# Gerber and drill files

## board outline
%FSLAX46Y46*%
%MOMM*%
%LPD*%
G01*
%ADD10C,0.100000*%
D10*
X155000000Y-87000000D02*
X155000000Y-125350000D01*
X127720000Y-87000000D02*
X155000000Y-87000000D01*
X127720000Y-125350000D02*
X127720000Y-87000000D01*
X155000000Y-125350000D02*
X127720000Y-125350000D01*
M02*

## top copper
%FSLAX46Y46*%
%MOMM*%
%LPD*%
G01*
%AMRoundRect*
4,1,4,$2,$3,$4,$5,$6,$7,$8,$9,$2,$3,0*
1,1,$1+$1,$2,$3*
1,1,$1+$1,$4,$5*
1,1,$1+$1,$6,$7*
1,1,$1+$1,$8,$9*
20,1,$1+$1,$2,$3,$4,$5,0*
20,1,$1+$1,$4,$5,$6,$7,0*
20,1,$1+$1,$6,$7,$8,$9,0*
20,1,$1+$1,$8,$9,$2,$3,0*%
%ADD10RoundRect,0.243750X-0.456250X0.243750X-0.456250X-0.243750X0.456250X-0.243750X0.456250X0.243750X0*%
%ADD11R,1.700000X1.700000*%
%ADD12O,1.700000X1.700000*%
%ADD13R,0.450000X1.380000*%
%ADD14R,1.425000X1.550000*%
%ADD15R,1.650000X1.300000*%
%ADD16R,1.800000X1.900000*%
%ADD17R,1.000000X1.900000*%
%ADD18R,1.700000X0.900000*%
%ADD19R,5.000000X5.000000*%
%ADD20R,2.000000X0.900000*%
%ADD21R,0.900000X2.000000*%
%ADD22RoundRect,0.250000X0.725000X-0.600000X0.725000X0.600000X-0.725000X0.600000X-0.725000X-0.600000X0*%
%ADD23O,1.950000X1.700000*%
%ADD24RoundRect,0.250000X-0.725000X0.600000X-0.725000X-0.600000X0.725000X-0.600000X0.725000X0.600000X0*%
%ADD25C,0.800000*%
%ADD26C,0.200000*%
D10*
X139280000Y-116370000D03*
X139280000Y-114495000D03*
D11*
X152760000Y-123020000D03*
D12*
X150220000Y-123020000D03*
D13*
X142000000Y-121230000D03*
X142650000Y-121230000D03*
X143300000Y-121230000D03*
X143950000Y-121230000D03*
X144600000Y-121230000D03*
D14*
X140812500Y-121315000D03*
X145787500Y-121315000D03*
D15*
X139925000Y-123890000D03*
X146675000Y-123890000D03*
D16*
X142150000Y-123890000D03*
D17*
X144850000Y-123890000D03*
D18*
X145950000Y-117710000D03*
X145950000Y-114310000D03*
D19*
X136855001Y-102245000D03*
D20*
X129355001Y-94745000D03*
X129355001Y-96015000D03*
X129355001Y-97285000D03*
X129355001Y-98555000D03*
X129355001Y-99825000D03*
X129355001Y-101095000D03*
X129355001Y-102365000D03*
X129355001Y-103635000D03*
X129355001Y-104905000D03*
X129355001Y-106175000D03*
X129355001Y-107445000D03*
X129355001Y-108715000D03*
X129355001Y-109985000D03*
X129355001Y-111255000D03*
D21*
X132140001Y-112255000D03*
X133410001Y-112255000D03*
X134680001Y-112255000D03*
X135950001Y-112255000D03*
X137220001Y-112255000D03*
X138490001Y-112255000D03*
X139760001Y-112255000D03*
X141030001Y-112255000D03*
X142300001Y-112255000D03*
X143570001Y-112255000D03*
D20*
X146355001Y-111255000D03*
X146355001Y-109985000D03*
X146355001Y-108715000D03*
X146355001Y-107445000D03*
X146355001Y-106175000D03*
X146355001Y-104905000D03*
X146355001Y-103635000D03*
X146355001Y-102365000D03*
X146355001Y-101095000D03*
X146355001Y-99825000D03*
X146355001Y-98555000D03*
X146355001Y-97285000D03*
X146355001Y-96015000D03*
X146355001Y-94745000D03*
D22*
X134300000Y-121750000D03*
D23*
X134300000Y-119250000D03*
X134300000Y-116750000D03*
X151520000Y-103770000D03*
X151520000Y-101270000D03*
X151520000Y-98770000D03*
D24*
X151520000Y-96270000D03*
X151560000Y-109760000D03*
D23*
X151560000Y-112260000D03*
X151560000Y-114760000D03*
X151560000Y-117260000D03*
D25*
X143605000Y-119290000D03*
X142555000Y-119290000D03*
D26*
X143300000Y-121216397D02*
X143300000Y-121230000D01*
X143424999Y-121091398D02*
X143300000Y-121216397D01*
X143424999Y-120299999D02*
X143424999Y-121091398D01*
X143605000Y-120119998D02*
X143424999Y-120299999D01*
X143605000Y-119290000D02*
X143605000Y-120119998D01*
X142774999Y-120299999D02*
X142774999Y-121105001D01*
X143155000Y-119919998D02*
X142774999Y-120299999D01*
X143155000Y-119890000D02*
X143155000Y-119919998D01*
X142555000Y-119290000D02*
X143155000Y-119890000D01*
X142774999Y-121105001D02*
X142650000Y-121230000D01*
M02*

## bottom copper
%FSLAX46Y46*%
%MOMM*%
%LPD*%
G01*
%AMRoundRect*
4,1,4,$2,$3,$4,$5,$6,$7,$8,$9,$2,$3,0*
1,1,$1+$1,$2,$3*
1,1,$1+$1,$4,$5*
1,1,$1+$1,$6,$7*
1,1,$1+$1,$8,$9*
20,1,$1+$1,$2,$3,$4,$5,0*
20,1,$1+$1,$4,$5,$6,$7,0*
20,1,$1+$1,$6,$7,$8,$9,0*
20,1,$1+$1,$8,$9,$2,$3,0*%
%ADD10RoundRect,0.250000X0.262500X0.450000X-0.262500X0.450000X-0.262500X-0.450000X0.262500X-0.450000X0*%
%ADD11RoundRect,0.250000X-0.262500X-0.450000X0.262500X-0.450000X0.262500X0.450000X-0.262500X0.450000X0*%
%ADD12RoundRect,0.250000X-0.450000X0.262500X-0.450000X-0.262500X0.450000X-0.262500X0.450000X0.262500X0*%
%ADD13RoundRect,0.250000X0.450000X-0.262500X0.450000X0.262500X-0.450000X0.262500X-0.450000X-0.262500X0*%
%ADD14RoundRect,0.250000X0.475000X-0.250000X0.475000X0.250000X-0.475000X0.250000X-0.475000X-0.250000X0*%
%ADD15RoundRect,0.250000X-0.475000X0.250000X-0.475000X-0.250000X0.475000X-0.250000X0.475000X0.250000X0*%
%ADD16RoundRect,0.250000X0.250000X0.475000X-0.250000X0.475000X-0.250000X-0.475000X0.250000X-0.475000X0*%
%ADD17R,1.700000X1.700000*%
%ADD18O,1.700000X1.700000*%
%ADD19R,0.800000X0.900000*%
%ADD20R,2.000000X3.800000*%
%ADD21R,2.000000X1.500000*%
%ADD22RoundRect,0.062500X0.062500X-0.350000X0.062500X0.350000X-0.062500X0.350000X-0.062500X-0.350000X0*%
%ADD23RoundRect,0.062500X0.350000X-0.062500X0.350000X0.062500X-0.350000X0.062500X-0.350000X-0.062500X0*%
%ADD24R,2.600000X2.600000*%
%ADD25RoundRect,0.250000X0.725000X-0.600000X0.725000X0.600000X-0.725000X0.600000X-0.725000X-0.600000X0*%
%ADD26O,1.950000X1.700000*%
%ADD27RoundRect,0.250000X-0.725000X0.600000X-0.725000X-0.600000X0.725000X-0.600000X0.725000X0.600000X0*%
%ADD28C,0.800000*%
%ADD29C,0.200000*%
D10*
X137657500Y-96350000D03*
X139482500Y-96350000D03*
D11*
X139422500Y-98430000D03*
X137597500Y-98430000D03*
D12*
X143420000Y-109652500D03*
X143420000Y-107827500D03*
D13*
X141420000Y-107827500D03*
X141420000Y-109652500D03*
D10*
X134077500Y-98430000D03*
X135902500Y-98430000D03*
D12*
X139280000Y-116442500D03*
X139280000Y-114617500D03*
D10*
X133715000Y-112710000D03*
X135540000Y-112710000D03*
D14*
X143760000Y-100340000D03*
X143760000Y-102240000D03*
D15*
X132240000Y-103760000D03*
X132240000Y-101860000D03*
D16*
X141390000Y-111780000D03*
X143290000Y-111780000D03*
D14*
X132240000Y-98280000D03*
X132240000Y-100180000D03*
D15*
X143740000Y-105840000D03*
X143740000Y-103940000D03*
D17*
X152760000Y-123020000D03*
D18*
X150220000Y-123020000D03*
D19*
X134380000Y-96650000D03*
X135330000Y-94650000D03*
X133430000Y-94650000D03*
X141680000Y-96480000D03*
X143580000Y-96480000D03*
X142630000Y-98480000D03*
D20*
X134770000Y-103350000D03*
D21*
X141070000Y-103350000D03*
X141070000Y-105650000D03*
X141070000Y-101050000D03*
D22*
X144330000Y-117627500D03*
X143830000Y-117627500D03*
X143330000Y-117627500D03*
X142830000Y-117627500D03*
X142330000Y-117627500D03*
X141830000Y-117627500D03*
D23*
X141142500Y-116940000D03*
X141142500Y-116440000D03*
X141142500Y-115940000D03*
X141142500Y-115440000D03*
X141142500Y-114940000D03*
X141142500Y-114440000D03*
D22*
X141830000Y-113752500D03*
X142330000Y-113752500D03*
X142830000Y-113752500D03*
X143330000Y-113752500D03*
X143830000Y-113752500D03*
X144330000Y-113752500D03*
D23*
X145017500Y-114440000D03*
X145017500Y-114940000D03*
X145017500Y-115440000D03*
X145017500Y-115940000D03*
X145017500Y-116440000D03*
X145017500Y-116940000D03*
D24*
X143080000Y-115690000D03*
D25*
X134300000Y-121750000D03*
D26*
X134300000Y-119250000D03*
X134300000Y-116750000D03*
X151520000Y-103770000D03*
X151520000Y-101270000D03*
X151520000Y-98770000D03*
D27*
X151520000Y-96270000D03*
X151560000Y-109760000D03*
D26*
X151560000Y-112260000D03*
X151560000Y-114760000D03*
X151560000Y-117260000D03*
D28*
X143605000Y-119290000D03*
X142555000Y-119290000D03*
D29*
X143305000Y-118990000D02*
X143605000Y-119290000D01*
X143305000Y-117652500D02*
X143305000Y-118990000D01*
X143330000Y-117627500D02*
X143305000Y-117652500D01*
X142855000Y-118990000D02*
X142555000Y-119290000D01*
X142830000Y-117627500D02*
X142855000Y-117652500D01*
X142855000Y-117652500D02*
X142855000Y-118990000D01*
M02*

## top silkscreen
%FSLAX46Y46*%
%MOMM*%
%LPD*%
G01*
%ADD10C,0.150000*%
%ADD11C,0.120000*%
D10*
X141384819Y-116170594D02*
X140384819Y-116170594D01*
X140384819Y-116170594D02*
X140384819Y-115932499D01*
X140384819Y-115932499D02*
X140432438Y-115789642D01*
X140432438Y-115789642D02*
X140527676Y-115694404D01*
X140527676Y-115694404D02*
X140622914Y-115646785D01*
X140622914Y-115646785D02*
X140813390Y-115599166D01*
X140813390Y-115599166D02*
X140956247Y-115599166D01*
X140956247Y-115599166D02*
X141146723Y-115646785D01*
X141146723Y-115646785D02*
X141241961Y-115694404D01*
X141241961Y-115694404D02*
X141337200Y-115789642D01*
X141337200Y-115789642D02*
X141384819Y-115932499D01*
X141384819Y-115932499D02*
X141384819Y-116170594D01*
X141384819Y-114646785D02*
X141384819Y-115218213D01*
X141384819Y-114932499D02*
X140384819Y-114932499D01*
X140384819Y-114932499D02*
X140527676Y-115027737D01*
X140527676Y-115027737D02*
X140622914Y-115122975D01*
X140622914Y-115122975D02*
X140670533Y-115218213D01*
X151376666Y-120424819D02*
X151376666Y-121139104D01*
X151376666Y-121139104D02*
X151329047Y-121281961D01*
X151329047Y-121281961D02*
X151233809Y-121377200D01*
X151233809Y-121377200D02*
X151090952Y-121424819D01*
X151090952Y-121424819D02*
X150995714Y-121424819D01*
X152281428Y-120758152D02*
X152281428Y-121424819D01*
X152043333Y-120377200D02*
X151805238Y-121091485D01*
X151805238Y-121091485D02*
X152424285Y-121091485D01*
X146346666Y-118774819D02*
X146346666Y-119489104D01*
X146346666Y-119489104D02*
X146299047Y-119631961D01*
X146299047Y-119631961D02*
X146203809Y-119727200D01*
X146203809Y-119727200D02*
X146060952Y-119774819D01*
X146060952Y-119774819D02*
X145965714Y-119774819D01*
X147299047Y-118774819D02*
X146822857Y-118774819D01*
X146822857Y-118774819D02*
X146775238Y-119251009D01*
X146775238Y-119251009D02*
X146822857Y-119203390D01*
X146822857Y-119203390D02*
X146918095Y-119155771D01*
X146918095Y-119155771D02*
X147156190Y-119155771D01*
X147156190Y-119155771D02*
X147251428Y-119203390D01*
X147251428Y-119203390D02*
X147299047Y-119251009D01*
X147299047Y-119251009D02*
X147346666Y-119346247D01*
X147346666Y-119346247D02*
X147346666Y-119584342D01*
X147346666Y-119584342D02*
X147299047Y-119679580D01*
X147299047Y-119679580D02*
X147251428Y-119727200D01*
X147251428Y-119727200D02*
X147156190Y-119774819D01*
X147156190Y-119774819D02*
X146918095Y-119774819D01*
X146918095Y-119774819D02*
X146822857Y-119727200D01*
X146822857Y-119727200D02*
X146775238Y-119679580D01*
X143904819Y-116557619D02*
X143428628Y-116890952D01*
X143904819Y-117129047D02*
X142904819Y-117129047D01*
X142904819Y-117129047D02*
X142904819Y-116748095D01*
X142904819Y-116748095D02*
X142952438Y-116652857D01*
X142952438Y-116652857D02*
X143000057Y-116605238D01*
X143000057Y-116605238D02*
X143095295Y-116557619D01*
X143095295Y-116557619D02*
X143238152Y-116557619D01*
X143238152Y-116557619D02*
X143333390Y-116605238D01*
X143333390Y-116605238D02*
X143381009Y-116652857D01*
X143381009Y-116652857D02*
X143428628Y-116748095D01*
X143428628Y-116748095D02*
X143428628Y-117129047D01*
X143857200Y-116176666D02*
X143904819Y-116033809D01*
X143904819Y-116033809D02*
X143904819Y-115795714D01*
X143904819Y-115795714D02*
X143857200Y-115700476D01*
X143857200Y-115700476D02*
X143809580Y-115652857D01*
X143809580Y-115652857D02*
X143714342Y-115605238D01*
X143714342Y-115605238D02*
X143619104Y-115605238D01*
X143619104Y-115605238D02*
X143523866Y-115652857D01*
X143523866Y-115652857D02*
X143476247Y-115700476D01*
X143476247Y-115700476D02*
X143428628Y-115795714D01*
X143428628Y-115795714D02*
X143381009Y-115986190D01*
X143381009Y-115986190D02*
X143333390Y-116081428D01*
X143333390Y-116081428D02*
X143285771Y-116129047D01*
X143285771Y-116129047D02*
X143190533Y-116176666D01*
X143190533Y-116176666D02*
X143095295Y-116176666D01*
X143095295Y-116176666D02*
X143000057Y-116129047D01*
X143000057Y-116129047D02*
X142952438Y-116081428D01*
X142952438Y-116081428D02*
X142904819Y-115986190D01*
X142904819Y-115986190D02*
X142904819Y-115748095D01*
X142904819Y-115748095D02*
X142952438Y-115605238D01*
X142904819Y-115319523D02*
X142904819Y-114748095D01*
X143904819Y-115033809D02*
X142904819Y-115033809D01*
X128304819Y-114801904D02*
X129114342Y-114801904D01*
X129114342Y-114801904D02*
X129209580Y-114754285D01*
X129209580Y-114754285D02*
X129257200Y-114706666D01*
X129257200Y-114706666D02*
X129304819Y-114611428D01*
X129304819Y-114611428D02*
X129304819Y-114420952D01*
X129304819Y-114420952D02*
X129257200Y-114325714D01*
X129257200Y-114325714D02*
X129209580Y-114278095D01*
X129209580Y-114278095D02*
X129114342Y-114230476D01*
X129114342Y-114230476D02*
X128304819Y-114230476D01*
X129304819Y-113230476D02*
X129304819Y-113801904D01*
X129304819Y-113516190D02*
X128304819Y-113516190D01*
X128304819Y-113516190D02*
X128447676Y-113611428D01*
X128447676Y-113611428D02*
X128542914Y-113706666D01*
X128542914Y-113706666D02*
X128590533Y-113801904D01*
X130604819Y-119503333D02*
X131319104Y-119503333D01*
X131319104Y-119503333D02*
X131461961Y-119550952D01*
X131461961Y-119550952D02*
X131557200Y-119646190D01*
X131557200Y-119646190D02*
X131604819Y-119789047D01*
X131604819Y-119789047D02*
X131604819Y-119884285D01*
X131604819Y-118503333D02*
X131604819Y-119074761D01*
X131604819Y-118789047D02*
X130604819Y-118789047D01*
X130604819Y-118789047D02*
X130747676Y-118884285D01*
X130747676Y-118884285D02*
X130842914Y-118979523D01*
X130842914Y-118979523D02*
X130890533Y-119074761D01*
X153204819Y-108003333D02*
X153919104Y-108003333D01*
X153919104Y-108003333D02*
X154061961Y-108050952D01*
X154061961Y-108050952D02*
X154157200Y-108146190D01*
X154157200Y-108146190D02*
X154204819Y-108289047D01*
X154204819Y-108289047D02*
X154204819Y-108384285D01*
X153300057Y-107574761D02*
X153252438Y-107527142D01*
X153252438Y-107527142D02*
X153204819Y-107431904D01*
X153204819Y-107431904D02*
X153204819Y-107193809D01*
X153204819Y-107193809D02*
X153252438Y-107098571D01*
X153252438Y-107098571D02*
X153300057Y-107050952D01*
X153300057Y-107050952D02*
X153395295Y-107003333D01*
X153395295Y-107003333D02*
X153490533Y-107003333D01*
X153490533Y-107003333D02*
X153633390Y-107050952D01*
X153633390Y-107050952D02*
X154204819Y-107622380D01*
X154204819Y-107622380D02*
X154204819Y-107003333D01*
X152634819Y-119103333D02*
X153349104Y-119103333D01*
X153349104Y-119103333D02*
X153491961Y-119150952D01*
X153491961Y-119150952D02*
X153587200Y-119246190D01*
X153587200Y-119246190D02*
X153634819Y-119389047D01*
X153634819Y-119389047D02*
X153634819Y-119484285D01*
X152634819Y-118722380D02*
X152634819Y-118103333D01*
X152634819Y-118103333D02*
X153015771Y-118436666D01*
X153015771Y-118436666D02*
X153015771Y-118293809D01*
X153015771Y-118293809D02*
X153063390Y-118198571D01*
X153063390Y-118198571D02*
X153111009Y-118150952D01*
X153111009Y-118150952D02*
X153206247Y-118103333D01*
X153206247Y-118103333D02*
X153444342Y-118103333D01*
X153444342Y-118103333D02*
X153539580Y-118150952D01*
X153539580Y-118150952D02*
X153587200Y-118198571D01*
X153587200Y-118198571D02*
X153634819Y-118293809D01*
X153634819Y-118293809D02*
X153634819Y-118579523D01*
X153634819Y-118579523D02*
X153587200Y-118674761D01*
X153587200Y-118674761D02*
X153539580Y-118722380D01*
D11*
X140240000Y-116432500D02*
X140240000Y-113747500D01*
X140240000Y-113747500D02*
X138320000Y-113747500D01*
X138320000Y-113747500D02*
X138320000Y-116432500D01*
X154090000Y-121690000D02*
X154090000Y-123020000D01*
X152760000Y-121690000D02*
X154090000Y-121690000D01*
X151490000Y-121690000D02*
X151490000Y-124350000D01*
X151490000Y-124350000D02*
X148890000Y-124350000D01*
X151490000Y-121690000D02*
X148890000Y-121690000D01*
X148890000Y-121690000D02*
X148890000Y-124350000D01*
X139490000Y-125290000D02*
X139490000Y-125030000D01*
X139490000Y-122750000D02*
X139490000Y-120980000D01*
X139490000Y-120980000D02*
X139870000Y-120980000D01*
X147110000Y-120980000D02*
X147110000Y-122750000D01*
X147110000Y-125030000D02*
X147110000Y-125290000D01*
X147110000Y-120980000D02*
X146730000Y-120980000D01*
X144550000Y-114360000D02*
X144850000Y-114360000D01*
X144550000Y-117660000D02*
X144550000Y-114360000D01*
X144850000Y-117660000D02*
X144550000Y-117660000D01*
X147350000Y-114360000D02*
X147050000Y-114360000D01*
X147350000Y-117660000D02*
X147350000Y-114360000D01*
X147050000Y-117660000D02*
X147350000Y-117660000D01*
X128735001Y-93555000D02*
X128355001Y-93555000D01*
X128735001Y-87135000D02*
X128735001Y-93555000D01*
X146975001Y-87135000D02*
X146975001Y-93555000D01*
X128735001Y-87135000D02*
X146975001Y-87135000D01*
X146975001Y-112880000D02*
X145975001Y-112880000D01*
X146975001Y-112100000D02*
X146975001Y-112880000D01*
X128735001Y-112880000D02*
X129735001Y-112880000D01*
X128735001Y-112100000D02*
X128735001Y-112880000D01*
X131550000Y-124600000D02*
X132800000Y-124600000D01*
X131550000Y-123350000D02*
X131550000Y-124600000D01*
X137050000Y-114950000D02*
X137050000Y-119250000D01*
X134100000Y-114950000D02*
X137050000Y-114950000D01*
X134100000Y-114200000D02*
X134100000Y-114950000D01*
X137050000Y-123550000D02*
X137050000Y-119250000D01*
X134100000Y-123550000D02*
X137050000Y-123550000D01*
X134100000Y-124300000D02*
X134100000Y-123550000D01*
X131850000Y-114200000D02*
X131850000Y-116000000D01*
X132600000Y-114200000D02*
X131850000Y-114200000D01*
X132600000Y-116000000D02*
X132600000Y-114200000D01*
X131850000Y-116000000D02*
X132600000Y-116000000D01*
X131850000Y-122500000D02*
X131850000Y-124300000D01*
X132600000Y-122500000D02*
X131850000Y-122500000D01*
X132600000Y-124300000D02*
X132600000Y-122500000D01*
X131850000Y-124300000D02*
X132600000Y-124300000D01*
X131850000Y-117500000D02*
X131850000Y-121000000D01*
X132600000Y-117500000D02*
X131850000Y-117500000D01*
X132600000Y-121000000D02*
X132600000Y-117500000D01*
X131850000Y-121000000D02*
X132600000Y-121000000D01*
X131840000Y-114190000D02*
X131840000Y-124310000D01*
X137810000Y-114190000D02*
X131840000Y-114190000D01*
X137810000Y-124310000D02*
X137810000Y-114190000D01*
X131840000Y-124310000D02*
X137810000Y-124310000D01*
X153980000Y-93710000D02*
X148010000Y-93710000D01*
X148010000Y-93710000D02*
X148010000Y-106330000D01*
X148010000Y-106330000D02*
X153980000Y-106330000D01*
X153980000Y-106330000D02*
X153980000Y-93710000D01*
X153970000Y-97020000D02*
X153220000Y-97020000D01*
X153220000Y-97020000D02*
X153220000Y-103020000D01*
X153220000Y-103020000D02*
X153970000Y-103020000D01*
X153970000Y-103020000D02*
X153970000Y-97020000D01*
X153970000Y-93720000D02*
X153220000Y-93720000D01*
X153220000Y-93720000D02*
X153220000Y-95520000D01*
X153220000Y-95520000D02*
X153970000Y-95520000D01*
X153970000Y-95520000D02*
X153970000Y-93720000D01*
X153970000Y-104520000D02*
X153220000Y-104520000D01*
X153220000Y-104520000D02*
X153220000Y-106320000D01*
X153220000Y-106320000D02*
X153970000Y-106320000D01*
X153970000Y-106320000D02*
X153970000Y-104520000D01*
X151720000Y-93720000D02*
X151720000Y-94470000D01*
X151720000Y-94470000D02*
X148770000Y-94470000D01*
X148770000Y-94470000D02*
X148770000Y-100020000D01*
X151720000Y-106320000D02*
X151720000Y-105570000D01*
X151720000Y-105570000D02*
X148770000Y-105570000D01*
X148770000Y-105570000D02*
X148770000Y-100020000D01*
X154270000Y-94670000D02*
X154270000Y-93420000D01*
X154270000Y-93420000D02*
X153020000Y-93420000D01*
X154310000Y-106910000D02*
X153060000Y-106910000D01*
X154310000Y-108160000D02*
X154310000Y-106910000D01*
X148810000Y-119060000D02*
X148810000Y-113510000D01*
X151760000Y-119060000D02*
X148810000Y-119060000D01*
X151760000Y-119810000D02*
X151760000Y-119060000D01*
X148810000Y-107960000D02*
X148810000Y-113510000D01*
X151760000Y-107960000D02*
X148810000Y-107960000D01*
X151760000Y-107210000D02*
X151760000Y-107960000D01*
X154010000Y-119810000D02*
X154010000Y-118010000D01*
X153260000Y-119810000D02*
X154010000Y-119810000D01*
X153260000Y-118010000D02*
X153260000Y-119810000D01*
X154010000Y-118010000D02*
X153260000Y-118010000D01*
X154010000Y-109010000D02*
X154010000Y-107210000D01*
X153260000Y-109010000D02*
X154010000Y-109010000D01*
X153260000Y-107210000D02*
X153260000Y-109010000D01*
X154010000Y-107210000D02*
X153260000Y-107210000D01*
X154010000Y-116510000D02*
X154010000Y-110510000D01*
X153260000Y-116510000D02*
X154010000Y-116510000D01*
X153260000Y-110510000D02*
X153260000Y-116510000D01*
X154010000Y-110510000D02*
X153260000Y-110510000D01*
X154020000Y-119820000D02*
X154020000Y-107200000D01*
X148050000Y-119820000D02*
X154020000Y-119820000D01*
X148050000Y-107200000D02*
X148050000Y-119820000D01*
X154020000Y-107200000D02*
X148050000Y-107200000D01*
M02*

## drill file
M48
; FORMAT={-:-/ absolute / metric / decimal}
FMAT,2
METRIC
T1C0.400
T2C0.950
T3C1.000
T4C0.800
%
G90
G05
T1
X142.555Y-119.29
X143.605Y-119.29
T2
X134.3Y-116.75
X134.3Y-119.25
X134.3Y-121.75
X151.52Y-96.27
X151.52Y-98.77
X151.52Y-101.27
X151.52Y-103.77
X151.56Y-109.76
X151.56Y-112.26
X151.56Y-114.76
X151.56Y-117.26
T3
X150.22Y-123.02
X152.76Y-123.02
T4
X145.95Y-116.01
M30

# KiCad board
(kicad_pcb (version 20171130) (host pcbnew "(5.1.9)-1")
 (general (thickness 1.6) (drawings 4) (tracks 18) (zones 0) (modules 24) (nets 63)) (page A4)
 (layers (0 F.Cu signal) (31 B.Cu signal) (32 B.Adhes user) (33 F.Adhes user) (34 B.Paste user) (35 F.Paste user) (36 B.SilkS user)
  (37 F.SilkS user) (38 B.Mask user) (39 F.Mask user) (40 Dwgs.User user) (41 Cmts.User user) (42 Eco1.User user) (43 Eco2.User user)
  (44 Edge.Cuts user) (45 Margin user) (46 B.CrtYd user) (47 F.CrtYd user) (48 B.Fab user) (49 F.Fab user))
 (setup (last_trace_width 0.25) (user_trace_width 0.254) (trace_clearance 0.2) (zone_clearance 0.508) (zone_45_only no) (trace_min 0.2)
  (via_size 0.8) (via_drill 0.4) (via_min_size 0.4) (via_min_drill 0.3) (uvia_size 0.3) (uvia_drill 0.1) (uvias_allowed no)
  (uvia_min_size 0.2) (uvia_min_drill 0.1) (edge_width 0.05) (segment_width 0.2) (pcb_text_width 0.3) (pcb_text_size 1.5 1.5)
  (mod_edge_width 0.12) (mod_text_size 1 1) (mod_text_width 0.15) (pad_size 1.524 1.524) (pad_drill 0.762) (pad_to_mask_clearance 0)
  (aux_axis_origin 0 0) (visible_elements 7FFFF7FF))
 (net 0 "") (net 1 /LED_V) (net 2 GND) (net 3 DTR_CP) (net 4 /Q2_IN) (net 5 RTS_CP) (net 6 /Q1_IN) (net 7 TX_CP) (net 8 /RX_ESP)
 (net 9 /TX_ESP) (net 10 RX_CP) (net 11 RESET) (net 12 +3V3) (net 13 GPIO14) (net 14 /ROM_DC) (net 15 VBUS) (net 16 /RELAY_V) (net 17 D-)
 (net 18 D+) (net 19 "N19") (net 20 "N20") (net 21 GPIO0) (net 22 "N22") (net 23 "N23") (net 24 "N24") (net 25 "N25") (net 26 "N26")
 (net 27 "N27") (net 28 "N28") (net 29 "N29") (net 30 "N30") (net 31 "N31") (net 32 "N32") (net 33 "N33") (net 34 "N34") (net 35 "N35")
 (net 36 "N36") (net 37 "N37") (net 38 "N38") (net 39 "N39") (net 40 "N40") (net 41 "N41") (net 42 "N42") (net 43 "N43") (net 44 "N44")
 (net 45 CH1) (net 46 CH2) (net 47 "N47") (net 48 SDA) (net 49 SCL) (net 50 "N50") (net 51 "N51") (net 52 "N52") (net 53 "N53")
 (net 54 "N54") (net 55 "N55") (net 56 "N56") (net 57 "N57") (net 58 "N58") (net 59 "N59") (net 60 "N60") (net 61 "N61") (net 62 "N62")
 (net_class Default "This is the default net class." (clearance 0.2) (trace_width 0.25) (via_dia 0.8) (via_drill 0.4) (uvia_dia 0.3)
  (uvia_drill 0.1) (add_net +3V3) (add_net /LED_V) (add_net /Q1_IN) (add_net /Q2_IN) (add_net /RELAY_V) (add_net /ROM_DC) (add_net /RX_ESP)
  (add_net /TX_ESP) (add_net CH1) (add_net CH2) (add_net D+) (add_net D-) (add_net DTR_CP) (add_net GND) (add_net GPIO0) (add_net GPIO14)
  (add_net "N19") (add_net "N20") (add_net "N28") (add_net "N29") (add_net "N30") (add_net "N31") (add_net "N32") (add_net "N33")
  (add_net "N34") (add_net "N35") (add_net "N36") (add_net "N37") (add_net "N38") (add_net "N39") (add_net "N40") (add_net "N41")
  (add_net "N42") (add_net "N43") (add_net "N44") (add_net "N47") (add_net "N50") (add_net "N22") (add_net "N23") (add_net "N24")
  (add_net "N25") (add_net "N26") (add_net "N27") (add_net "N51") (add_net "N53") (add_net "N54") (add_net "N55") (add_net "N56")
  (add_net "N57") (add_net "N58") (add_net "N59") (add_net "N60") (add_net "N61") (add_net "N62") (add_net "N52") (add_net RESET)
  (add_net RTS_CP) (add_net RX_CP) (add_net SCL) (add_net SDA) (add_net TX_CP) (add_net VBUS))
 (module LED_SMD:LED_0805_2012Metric (layer F.Cu) (at 139.28 115.4325 270)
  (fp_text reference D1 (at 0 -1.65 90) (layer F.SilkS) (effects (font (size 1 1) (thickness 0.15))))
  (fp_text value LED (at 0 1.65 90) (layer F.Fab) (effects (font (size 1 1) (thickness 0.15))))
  (fp_line (start 1 -0.96) (end -1.685 -0.96) (layer F.SilkS) (width 0.12))
  (fp_line (start -1.685 -0.96) (end -1.685 0.96) (layer F.SilkS) (width 0.12))
  (fp_line (start -1.685 0.96) (end 1 0.96) (layer F.SilkS) (width 0.12))
  (pad 2 smd roundrect (at 0.9375 0 270) (size 0.975 1.4) (layers F.Cu F.Paste F.Mask) (roundrect_rratio 0.25) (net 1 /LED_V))
  (pad 1 smd roundrect (at -0.9375 0 270) (size 0.975 1.4) (layers F.Cu F.Paste F.Mask) (roundrect_rratio 0.25) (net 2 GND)))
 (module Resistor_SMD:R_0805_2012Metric (layer B.Cu) (at 138.57 96.35 180)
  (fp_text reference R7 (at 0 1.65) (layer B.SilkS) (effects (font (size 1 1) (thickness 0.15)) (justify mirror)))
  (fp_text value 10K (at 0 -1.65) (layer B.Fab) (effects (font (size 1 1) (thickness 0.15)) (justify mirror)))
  (pad 2 smd roundrect (at 0.9125 0 180) (size 1.025 1.4) (layers B.Cu B.Paste B.Mask) (roundrect_rratio 0.243902) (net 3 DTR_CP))
  (pad 1 smd roundrect (at -0.9125 0 180) (size 1.025 1.4) (layers B.Cu B.Paste B.Mask) (roundrect_rratio 0.243902) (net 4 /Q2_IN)))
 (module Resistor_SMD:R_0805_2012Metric (layer B.Cu) (at 138.51 98.43)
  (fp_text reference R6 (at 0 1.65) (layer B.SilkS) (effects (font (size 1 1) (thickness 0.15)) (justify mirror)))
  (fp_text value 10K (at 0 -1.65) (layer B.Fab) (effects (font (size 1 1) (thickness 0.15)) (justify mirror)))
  (pad 2 smd roundrect (at 0.9125 0) (size 1.025 1.4) (layers B.Cu B.Paste B.Mask) (roundrect_rratio 0.243902) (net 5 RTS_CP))
  (pad 1 smd roundrect (at -0.9125 0) (size 1.025 1.4) (layers B.Cu B.Paste B.Mask) (roundrect_rratio 0.243902) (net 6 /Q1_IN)))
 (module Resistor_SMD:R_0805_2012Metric (layer B.Cu) (at 143.42 108.74 270)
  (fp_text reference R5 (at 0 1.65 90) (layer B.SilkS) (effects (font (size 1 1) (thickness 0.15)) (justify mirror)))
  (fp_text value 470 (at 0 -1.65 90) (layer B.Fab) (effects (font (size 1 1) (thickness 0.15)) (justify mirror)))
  (pad 2 smd roundrect (at 0.9125 0 270) (size 1.025 1.4) (layers B.Cu B.Paste B.Mask) (roundrect_rratio 0.243902) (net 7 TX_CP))
  (pad 1 smd roundrect (at -0.9125 0 270) (size 1.025 1.4) (layers B.Cu B.Paste B.Mask) (roundrect_rratio 0.243902) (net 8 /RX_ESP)))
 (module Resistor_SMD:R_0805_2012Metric (layer B.Cu) (at 141.42 108.74 90)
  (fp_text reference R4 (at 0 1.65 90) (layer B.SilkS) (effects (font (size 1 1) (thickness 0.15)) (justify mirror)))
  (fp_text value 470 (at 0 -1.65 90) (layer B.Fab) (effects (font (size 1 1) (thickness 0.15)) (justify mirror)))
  (pad 2 smd roundrect (at 0.9125 0 90) (size 1.025 1.4) (layers B.Cu B.Paste B.Mask) (roundrect_rratio 0.243902) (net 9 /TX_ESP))
  (pad 1 smd roundrect (at -0.9125 0 90) (size 1.025 1.4) (layers B.Cu B.Paste B.Mask) (roundrect_rratio 0.243902) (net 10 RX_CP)))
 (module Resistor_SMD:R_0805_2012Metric (layer B.Cu) (at 134.99 98.43 180)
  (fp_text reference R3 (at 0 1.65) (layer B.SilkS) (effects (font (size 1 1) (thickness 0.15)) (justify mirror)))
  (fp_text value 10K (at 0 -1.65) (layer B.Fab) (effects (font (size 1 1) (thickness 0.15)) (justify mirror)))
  (pad 2 smd roundrect (at 0.9125 0 180) (size 1.025 1.4) (layers B.Cu B.Paste B.Mask) (roundrect_rratio 0.243902) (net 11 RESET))
  (pad 1 smd roundrect (at -0.9125 0 180) (size 1.025 1.4) (layers B.Cu B.Paste B.Mask) (roundrect_rratio 0.243902) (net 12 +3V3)))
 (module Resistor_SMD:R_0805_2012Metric (layer B.Cu) (at 139.28 115.53 270)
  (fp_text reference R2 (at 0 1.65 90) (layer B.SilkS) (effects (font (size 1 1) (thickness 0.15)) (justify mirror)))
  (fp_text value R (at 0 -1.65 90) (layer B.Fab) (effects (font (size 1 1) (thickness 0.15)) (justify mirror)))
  (pad 2 smd roundrect (at 0.9125 0 270) (size 1.025 1.4) (layers B.Cu B.Paste B.Mask) (roundrect_rratio 0.243902) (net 1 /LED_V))
  (pad 1 smd roundrect (at -0.9125 0 270) (size 1.025 1.4) (layers B.Cu B.Paste B.Mask) (roundrect_rratio 0.243902) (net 12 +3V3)))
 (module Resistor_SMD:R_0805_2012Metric (layer B.Cu) (at 134.6275 112.71 180)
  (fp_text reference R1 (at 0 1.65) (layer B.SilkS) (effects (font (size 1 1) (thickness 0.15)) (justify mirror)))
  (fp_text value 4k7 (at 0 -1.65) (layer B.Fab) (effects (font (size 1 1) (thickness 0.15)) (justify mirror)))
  (pad 2 smd roundrect (at 0.9125 0 180) (size 1.025 1.4) (layers B.Cu B.Paste B.Mask) (roundrect_rratio 0.243902) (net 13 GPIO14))
  (pad 1 smd roundrect (at -0.9125 0 180) (size 1.025 1.4) (layers B.Cu B.Paste B.Mask) (roundrect_rratio 0.243902) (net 12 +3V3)))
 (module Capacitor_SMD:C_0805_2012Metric (layer B.Cu) (at 143.76 101.29 90)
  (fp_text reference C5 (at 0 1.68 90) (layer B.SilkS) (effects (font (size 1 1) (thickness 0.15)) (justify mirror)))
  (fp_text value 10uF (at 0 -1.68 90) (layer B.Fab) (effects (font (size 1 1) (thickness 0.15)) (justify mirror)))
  (pad 2 smd roundrect (at 0.95 0 90) (size 1 1.45) (layers B.Cu B.Paste B.Mask) (roundrect_rratio 0.25) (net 2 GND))
  (pad 1 smd roundrect (at -0.95 0 90) (size 1 1.45) (layers B.Cu B.Paste B.Mask) (roundrect_rratio 0.25) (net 12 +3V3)))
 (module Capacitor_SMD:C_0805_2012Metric (layer B.Cu) (at 132.24 102.81 270)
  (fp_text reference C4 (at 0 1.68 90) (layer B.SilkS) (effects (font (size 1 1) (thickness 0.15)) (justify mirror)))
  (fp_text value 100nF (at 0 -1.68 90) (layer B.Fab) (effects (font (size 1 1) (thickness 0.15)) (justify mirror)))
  (pad 2 smd roundrect (at 0.95 0 270) (size 1 1.45) (layers B.Cu B.Paste B.Mask) (roundrect_rratio 0.25) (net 12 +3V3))
  (pad 1 smd roundrect (at -0.95 0 270) (size 1 1.45) (layers B.Cu B.Paste B.Mask) (roundrect_rratio 0.25) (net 2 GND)))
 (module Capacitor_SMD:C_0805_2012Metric (layer B.Cu) (at 142.34 111.78 180)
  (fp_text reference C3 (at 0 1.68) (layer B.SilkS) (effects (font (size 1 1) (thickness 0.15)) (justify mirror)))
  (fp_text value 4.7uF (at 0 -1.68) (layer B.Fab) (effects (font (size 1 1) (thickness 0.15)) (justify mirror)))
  (pad 2 smd roundrect (at 0.95 0 180) (size 1 1.45) (layers B.Cu B.Paste B.Mask) (roundrect_rratio 0.25) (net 2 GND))
  (pad 1 smd roundrect (at -0.95 0 180) (size 1 1.45) (layers B.Cu B.Paste B.Mask) (roundrect_rratio 0.25) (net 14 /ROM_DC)))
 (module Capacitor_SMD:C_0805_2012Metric (layer B.Cu) (at 132.24 99.23 90)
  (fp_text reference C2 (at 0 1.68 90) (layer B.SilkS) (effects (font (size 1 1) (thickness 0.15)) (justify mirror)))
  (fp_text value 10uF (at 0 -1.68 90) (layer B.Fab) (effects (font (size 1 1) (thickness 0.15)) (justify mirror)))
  (pad 2 smd roundrect (at 0.95 0 90) (size 1 1.45) (layers B.Cu B.Paste B.Mask) (roundrect_rratio 0.25) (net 11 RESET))
  (pad 1 smd roundrect (at -0.95 0 90) (size 1 1.45) (layers B.Cu B.Paste B.Mask) (roundrect_rratio 0.25) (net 2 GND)))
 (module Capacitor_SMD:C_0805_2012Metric (layer B.Cu) (at 143.74 104.89 270)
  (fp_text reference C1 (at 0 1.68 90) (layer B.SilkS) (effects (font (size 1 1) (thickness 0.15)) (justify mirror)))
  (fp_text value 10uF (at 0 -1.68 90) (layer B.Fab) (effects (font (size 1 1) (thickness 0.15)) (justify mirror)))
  (pad 2 smd roundrect (at 0.95 0 270) (size 1 1.45) (layers B.Cu B.Paste B.Mask) (roundrect_rratio 0.25) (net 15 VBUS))
  (pad 1 smd roundrect (at -0.95 0 270) (size 1 1.45) (layers B.Cu B.Paste B.Mask) (roundrect_rratio 0.25) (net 2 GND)))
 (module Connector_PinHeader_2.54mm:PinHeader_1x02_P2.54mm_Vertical (layer F.Cu) (at 152.76 123.02 270)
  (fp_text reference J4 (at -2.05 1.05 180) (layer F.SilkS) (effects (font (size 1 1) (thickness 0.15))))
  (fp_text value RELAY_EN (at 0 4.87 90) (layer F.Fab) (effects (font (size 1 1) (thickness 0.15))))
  (fp_line (start -1.33 -1.33) (end 0 -1.33) (layer F.SilkS) (width 0.12))
  (fp_line (start -1.33 0) (end -1.33 -1.33) (layer F.SilkS) (width 0.12))
  (fp_line (start -1.33 1.27) (end 1.33 1.27) (layer F.SilkS) (width 0.12))
  (fp_line (start 1.33 1.27) (end 1.33 3.87) (layer F.SilkS) (width 0.12))
  (fp_line (start -1.33 1.27) (end -1.33 3.87) (layer F.SilkS) (width 0.12))
  (fp_line (start -1.33 3.87) (end 1.33 3.87) (layer F.SilkS) (width 0.12))
  (pad 1 thru_hole rect (at 0 0 270) (size 1.7 1.7) (drill 1) (layers *.Cu *.Mask) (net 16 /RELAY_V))
  (pad 2 thru_hole oval (at 0 2.54 270) (size 1.7 1.7) (drill 1) (layers *.Cu *.Mask) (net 15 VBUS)))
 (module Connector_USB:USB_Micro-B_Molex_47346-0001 (layer F.Cu) (at 143.3 122.69)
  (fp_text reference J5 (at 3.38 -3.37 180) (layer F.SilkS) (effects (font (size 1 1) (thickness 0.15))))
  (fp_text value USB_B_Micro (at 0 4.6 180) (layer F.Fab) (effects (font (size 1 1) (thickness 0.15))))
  (fp_line (start -3.81 2.6) (end -3.81 2.34) (layer F.SilkS) (width 0.12))
  (fp_line (start -3.81 0.06) (end -3.81 -1.71) (layer F.SilkS) (width 0.12))
  (fp_line (start -3.81 -1.71) (end -3.43 -1.71) (layer F.SilkS) (width 0.12))
  (fp_line (start 3.81 -1.71) (end 3.81 0.06) (layer F.SilkS) (width 0.12))
  (fp_line (start 3.81 2.34) (end 3.81 2.6) (layer F.SilkS) (width 0.12))
  (fp_line (start 3.81 -1.71) (end 3.43 -1.71) (layer F.SilkS) (width 0.12))
  (pad 1 smd rect (at -1.3 -1.46) (size 0.45 1.38) (layers F.Cu F.Paste F.Mask) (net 15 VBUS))
  (pad 2 smd rect (at -0.65 -1.46) (size 0.45 1.38) (layers F.Cu F.Paste F.Mask) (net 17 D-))
  (pad 3 smd rect (at 0 -1.46) (size 0.45 1.38) (layers F.Cu F.Paste F.Mask) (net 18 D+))
  (pad 4 smd rect (at 0.65 -1.46) (size 0.45 1.38) (layers F.Cu F.Paste F.Mask) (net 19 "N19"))
  (pad 5 smd rect (at 1.3 -1.46) (size 0.45 1.38) (layers F.Cu F.Paste F.Mask) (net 2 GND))
  (pad 6 smd rect (at -2.4875 -1.375) (size 1.425 1.55) (layers F.Cu F.Paste F.Mask) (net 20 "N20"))
  (pad 6 smd rect (at 2.4875 -1.375) (size 1.425 1.55) (layers F.Cu F.Paste F.Mask) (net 20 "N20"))
  (pad 6 smd rect (at -3.375 1.2) (size 1.65 1.3) (layers F.Cu F.Paste F.Mask) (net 20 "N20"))
  (pad 6 smd rect (at 3.375 1.2) (size 1.65 1.3) (layers F.Cu F.Paste F.Mask) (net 20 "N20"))
  (pad 6 smd rect (at -1.15 1.2) (size 1.8 1.9) (layers F.Cu F.Paste F.Mask) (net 20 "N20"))
  (pad 6 smd rect (at 1.55 1.2) (size 1 1.9) (layers F.Cu F.Paste F.Mask) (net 20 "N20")))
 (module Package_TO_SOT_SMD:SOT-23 (layer B.Cu) (at 134.38 95.65 270)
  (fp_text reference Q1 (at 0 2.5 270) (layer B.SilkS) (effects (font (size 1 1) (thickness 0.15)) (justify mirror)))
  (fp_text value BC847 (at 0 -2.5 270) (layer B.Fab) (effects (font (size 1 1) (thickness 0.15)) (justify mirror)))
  (pad 3 smd rect (at 1 0 270) (size 0.9 0.8) (layers B.Cu B.Paste B.Mask) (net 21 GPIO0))
  (pad 2 smd rect (at -1 -0.95 270) (size 0.9 0.8) (layers B.Cu B.Paste B.Mask) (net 3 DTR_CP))
  (pad 1 smd rect (at -1 0.95 270) (size 0.9 0.8) (layers B.Cu B.Paste B.Mask) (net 6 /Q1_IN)))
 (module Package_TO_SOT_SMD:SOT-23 (layer B.Cu) (at 142.63 97.48 270)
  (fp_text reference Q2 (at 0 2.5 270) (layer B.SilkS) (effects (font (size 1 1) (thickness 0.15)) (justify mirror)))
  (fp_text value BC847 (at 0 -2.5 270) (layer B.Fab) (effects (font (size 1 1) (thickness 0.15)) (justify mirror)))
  (pad 1 smd rect (at -1 0.95 270) (size 0.9 0.8) (layers B.Cu B.Paste B.Mask) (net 4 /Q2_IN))
  (pad 2 smd rect (at -1 -0.95 270) (size 0.9 0.8) (layers B.Cu B.Paste B.Mask) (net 11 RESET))
  (pad 3 smd rect (at 1 0 270) (size 0.9 0.8) (layers B.Cu B.Paste B.Mask) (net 5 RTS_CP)))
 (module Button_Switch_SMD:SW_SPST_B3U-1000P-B (layer F.Cu) (at 145.95 116.01 90)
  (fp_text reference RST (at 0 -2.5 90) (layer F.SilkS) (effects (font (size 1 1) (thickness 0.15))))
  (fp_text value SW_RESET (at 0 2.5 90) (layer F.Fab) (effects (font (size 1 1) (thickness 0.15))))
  (fp_line (start 1.65 -1.4) (end 1.65 -1.1) (layer F.SilkS) (width 0.12))
  (fp_line (start -1.65 -1.4) (end 1.65 -1.4) (layer F.SilkS) (width 0.12))
  (fp_line (start -1.65 -1.1) (end -1.65 -1.4) (layer F.SilkS) (width 0.12))
  (fp_line (start 1.65 1.4) (end 1.65 1.1) (layer F.SilkS) (width 0.12))
  (fp_line (start -1.65 1.4) (end 1.65 1.4) (layer F.SilkS) (width 0.12))
  (fp_line (start -1.65 1.1) (end -1.65 1.4) (layer F.SilkS) (width 0.12))
  (pad 1 smd rect (at -1.7 0 90) (size 0.9 1.7) (layers F.Cu F.Paste F.Mask) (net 2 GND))
  (pad 2 smd rect (at 1.7 0 90) (size 0.9 1.7) (layers F.Cu F.Paste F.Mask) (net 11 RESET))
  (pad "" np_thru_hole circle (at 0 0 90) (size 0.8 0.8) (drill 0.8) (layers *.Cu *.Mask)))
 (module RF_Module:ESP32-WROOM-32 (layer F.Cu) (at 137.855001 103)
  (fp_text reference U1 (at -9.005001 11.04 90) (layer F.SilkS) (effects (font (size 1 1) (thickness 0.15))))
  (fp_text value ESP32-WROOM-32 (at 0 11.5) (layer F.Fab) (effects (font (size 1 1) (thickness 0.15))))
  (fp_line (start -9.12 -9.445) (end -9.5 -9.445) (layer F.SilkS) (width 0.12))
  (fp_line (start -9.12 -15.865) (end -9.12 -9.445) (layer F.SilkS) (width 0.12))
  (fp_line (start 9.12 -15.865) (end 9.12 -9.445) (layer F.SilkS) (width 0.12))
  (fp_line (start -9.12 -15.865) (end 9.12 -15.865) (layer F.SilkS) (width 0.12))
  (fp_line (start 9.12 9.88) (end 8.12 9.88) (layer F.SilkS) (width 0.12))
  (fp_line (start 9.12 9.1) (end 9.12 9.88) (layer F.SilkS) (width 0.12))
  (fp_line (start -9.12 9.88) (end -8.12 9.88) (layer F.SilkS) (width 0.12))
  (fp_line (start -9.12 9.1) (end -9.12 9.88) (layer F.SilkS) (width 0.12))
  (pad 39 smd rect (at -1 -0.755) (size 5 5) (layers F.Cu F.Paste F.Mask) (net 2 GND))
  (pad 1 smd rect (at -8.5 -8.255) (size 2 0.9) (layers F.Cu F.Paste F.Mask) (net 2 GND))
  (pad 2 smd rect (at -8.5 -6.985) (size 2 0.9) (layers F.Cu F.Paste F.Mask) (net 12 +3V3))
  (pad 3 smd rect (at -8.5 -5.715) (size 2 0.9) (layers F.Cu F.Paste F.Mask) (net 11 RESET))
  (pad 4 smd rect (at -8.5 -4.445) (size 2 0.9) (layers F.Cu F.Paste F.Mask) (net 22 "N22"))
  (pad 5 smd rect (at -8.5 -3.175) (size 2 0.9) (layers F.Cu F.Paste F.Mask) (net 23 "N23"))
  (pad 6 smd rect (at -8.5 -1.905) (size 2 0.9) (layers F.Cu F.Paste F.Mask) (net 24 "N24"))
  (pad 7 smd rect (at -8.5 -0.635) (size 2 0.9) (layers F.Cu F.Paste F.Mask) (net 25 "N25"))
  (pad 8 smd rect (at -8.5 0.635) (size 2 0.9) (layers F.Cu F.Paste F.Mask) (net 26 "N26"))
  (pad 9 smd rect (at -8.5 1.905) (size 2 0.9) (layers F.Cu F.Paste F.Mask) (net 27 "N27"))
  (pad 10 smd rect (at -8.5 3.175) (size 2 0.9) (layers F.Cu F.Paste F.Mask) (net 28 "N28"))
  (pad 11 smd rect (at -8.5 4.445) (size 2 0.9) (layers F.Cu F.Paste F.Mask) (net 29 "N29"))
  (pad 12 smd rect (at -8.5 5.715) (size 2 0.9) (layers F.Cu F.Paste F.Mask) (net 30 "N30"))
  (pad 13 smd rect (at -8.5 6.985) (size 2 0.9) (layers F.Cu F.Paste F.Mask) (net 13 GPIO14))
  (pad 14 smd rect (at -8.5 8.255) (size 2 0.9) (layers F.Cu F.Paste F.Mask) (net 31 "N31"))
  (pad 15 smd rect (at -5.715 9.255 90) (size 2 0.9) (layers F.Cu F.Paste F.Mask) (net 2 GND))
  (pad 16 smd rect (at -4.445 9.255 90) (size 2 0.9) (layers F.Cu F.Paste F.Mask) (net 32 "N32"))
  (pad 17 smd rect (at -3.175 9.255 90) (size 2 0.9) (layers F.Cu F.Paste F.Mask) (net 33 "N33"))
  (pad 18 smd rect (at -1.905 9.255 90) (size 2 0.9) (layers F.Cu F.Paste F.Mask) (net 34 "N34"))
  (pad 19 smd rect (at -0.635 9.255 90) (size 2 0.9) (layers F.Cu F.Paste F.Mask) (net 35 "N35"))
  (pad 20 smd rect (at 0.635 9.255 90) (size 2 0.9) (layers F.Cu F.Paste F.Mask) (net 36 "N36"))
  (pad 21 smd rect (at 1.905 9.255 90) (size 2 0.9) (layers F.Cu F.Paste F.Mask) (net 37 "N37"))
  (pad 22 smd rect (at 3.175 9.255 90) (size 2 0.9) (layers F.Cu F.Paste F.Mask) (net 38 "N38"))
  (pad 23 smd rect (at 4.445 9.255 90) (size 2 0.9) (layers F.Cu F.Paste F.Mask) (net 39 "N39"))
  (pad 24 smd rect (at 5.715 9.255 90) (size 2 0.9) (layers F.Cu F.Paste F.Mask) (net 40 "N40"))
  (pad 25 smd rect (at 8.5 8.255) (size 2 0.9) (layers F.Cu F.Paste F.Mask) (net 21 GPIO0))
  (pad 26 smd rect (at 8.5 6.985) (size 2 0.9) (layers F.Cu F.Paste F.Mask) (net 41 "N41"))
  (pad 27 smd rect (at 8.5 5.715) (size 2 0.9) (layers F.Cu F.Paste F.Mask) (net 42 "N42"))
  (pad 28 smd rect (at 8.5 4.445) (size 2 0.9) (layers F.Cu F.Paste F.Mask) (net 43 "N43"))
  (pad 29 smd rect (at 8.5 3.175) (size 2 0.9) (layers F.Cu F.Paste F.Mask) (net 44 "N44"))
  (pad 30 smd rect (at 8.5 1.905) (size 2 0.9) (layers F.Cu F.Paste F.Mask) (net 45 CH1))
  (pad 31 smd rect (at 8.5 0.635) (size 2 0.9) (layers F.Cu F.Paste F.Mask) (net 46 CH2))
  (pad 32 smd rect (at 8.5 -0.635) (size 2 0.9) (layers F.Cu F.Paste F.Mask) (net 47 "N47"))
  (pad 33 smd rect (at 8.5 -1.905) (size 2 0.9) (layers F.Cu F.Paste F.Mask) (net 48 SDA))
  (pad 34 smd rect (at 8.5 -3.175) (size 2 0.9) (layers F.Cu F.Paste F.Mask) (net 8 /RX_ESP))
  (pad 35 smd rect (at 8.5 -4.445) (size 2 0.9) (layers F.Cu F.Paste F.Mask) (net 9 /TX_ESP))
  (pad 36 smd rect (at 8.5 -5.715) (size 2 0.9) (layers F.Cu F.Paste F.Mask) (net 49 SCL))
  (pad 37 smd rect (at 8.5 -6.985) (size 2 0.9) (layers F.Cu F.Paste F.Mask) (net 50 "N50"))
  (pad 38 smd rect (at 8.5 -8.255) (size 2 0.9) (layers F.Cu F.Paste F.Mask) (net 2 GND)))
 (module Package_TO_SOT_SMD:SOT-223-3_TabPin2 (layer B.Cu) (at 137.92 103.35 180)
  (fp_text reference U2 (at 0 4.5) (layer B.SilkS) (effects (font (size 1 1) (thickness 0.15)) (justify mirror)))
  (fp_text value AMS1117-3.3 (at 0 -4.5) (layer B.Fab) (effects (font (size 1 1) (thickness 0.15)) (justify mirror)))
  (pad 2 smd rect (at 3.15 0 180) (size 2 3.8) (layers B.Cu B.Paste B.Mask) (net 12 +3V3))
  (pad 2 smd rect (at -3.15 0 180) (size 2 1.5) (layers B.Cu B.Paste B.Mask) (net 12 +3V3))
  (pad 3 smd rect (at -3.15 -2.3 180) (size 2 1.5) (layers B.Cu B.Paste B.Mask) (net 15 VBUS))
  (pad 1 smd rect (at -3.15 2.3 180) (size 2 1.5) (layers B.Cu B.Paste B.Mask) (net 2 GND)))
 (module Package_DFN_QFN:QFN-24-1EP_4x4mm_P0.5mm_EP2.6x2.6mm (layer B.Cu) (at 143.08 115.69 90)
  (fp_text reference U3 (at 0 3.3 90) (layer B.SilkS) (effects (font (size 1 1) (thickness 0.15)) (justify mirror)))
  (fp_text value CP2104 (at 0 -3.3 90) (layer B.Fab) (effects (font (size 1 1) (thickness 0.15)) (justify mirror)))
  (pad 1 smd roundrect (at -1.9375 1.25 90) (size 0.825 0.25) (layers B.Cu B.Paste B.Mask) (roundrect_rratio 0.25) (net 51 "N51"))
  (pad 2 smd roundrect (at -1.9375 0.75 90) (size 0.825 0.25) (layers B.Cu B.Paste B.Mask) (roundrect_rratio 0.25) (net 2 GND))
  (pad 3 smd roundrect (at -1.9375 0.25 90) (size 0.825 0.25) (layers B.Cu B.Paste B.Mask) (roundrect_rratio 0.25) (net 18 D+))
  (pad 4 smd roundrect (at -1.9375 -0.25 90) (size 0.825 0.25) (layers B.Cu B.Paste B.Mask) (roundrect_rratio 0.25) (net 17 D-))
  (pad 5 smd roundrect (at -1.9375 -0.75 90) (size 0.825 0.25) (layers B.Cu B.Paste B.Mask) (roundrect_rratio 0.25) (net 12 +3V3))
  (pad 6 smd roundrect (at -1.9375 -1.25 90) (size 0.825 0.25) (layers B.Cu B.Paste B.Mask) (roundrect_rratio 0.25) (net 12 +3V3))
  (pad 7 smd roundrect (at -1.25 -1.9375 90) (size 0.25 0.825) (layers B.Cu B.Paste B.Mask) (roundrect_rratio 0.25) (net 12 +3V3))
  (pad 8 smd roundrect (at -0.75 -1.9375 90) (size 0.25 0.825) (layers B.Cu B.Paste B.Mask) (roundrect_rratio 0.25) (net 15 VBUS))
  (pad 9 smd roundrect (at -0.25 -1.9375 90) (size 0.25 0.825) (layers B.Cu B.Paste B.Mask) (roundrect_rratio 0.25) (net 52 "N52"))
  (pad 10 smd roundrect (at 0.25 -1.9375 90) (size 0.25 0.825) (layers B.Cu B.Paste B.Mask) (roundrect_rratio 0.25) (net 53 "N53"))
  (pad 11 smd roundrect (at 0.75 -1.9375 90) (size 0.25 0.825) (layers B.Cu B.Paste B.Mask) (roundrect_rratio 0.25) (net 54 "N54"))
  (pad 12 smd roundrect (at 1.25 -1.9375 90) (size 0.25 0.825) (layers B.Cu B.Paste B.Mask) (roundrect_rratio 0.25) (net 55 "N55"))
  (pad 13 smd roundrect (at 1.9375 -1.25 90) (size 0.825 0.25) (layers B.Cu B.Paste B.Mask) (roundrect_rratio 0.25) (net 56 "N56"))
  (pad 14 smd roundrect (at 1.9375 -0.75 90) (size 0.825 0.25) (layers B.Cu B.Paste B.Mask) (roundrect_rratio 0.25) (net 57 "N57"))
  (pad 15 smd roundrect (at 1.9375 -0.25 90) (size 0.825 0.25) (layers B.Cu B.Paste B.Mask) (roundrect_rratio 0.25) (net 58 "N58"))
  (pad 16 smd roundrect (at 1.9375 0.25 90) (size 0.825 0.25) (layers B.Cu B.Paste B.Mask) (roundrect_rratio 0.25) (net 14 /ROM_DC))
  (pad 17 smd roundrect (at 1.9375 0.75 90) (size 0.825 0.25) (layers B.Cu B.Paste B.Mask) (roundrect_rratio 0.25) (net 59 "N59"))
  (pad 18 smd roundrect (at 1.9375 1.25 90) (size 0.825 0.25) (layers B.Cu B.Paste B.Mask) (roundrect_rratio 0.25) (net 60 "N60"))
  (pad 19 smd roundrect (at 1.25 1.9375 90) (size 0.25 0.825) (layers B.Cu B.Paste B.Mask) (roundrect_rratio 0.25) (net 5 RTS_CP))
  (pad 20 smd roundrect (at 0.75 1.9375 90) (size 0.25 0.825) (layers B.Cu B.Paste B.Mask) (roundrect_rratio 0.25) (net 10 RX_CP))
  (pad 21 smd roundrect (at 0.25 1.9375 90) (size 0.25 0.825) (layers B.Cu B.Paste B.Mask) (roundrect_rratio 0.25) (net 7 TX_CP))
  (pad 22 smd roundrect (at -0.25 1.9375 90) (size 0.25 0.825) (layers B.Cu B.Paste B.Mask) (roundrect_rratio 0.25) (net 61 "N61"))
  (pad 23 smd roundrect (at -0.75 1.9375 90) (size 0.25 0.825) (layers B.Cu B.Paste B.Mask) (roundrect_rratio 0.25) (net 3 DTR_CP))
  (pad 24 smd roundrect (at -1.25 1.9375 90) (size 0.25 0.825) (layers B.Cu B.Paste B.Mask) (roundrect_rratio 0.25) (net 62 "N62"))
  (pad 25 smd rect (at 0 0 90) (size 2.6 2.6) (layers B.Cu B.Mask) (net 2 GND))
  (pad "" smd roundrect (at -0.65 0.65 90) (size 1.05 1.05) (layers B.Paste) (roundrect_rratio 0.238095))
  (pad "" smd roundrect (at -0.65 -0.65 90) (size 1.05 1.05) (layers B.Paste) (roundrect_rratio 0.238095))
  (pad "" smd roundrect (at 0.65 0.65 90) (size 1.05 1.05) (layers B.Paste) (roundrect_rratio 0.238095))
  (pad "" smd roundrect (at 0.65 -0.65 90) (size 1.05 1.05) (layers B.Paste) (roundrect_rratio 0.238095)))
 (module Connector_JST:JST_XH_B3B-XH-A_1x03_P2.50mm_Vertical (layer F.Cu) (at 134.3 121.75 90)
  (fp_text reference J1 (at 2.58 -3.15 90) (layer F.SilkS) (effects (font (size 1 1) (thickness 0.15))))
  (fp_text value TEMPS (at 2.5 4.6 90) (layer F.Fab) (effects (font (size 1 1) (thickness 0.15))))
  (fp_line (start -2.85 -2.75) (end -2.85 -1.5) (layer F.SilkS) (width 0.12))
  (fp_line (start -1.6 -2.75) (end -2.85 -2.75) (layer F.SilkS) (width 0.12))
  (fp_line (start 6.8 2.75) (end 2.5 2.75) (layer F.SilkS) (width 0.12))
  (fp_line (start 6.8 -0.2) (end 6.8 2.75) (layer F.SilkS) (width 0.12))
  (fp_line (start 7.55 -0.2) (end 6.8 -0.2) (layer F.SilkS) (width 0.12))
  (fp_line (start -1.8 2.75) (end 2.5 2.75) (layer F.SilkS) (width 0.12))
  (fp_line (start -1.8 -0.2) (end -1.8 2.75) (layer F.SilkS) (width 0.12))
  (fp_line (start -2.55 -0.2) (end -1.8 -0.2) (layer F.SilkS) (width 0.12))
  (fp_line (start 7.55 -2.45) (end 5.75 -2.45) (layer F.SilkS) (width 0.12))
  (fp_line (start 7.55 -1.7) (end 7.55 -2.45) (layer F.SilkS) (width 0.12))
  (fp_line (start 5.75 -1.7) (end 7.55 -1.7) (layer F.SilkS) (width 0.12))
  (fp_line (start 5.75 -2.45) (end 5.75 -1.7) (layer F.SilkS) (width 0.12))
  (fp_line (start -0.75 -2.45) (end -2.55 -2.45) (layer F.SilkS) (width 0.12))
  (fp_line (start -0.75 -1.7) (end -0.75 -2.45) (layer F.SilkS) (width 0.12))
  (fp_line (start -2.55 -1.7) (end -0.75 -1.7) (layer F.SilkS) (width 0.12))
  (fp_line (start -2.55 -2.45) (end -2.55 -1.7) (layer F.SilkS) (width 0.12))
  (fp_line (start 4.25 -2.45) (end 0.75 -2.45) (layer F.SilkS) (width 0.12))
  (fp_line (start 4.25 -1.7) (end 4.25 -2.45) (layer F.SilkS) (width 0.12))
  (fp_line (start 0.75 -1.7) (end 4.25 -1.7) (layer F.SilkS) (width 0.12))
  (fp_line (start 0.75 -2.45) (end 0.75 -1.7) (layer F.SilkS) (width 0.12))
  (fp_line (start 7.56 -2.46) (end -2.56 -2.46) (layer F.SilkS) (width 0.12))
  (fp_line (start 7.56 3.51) (end 7.56 -2.46) (layer F.SilkS) (width 0.12))
  (fp_line (start -2.56 3.51) (end 7.56 3.51) (layer F.SilkS) (width 0.12))
  (fp_line (start -2.56 -2.46) (end -2.56 3.51) (layer F.SilkS) (width 0.12))
  (pad 1 thru_hole roundrect (at 0 0 90) (size 1.7 1.95) (drill 0.95) (layers *.Cu *.Mask) (roundrect_rratio 0.147059) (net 13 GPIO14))
  (pad 2 thru_hole oval (at 2.5 0 90) (size 1.7 1.95) (drill 0.95) (layers *.Cu *.Mask) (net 12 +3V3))
  (pad 3 thru_hole oval (at 5 0 90) (size 1.7 1.95) (drill 0.95) (layers *.Cu *.Mask) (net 2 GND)))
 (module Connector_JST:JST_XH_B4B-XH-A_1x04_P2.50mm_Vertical (layer F.Cu) (at 151.52 96.27 270)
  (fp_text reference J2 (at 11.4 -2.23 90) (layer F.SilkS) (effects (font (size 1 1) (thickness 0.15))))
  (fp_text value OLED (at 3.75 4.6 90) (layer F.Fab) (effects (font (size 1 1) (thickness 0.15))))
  (fp_line (start -2.56 -2.46) (end -2.56 3.51) (layer F.SilkS) (width 0.12))
  (fp_line (start -2.56 3.51) (end 10.06 3.51) (layer F.SilkS) (width 0.12))
  (fp_line (start 10.06 3.51) (end 10.06 -2.46) (layer F.SilkS) (width 0.12))
  (fp_line (start 10.06 -2.46) (end -2.56 -2.46) (layer F.SilkS) (width 0.12))
  (fp_line (start 0.75 -2.45) (end 0.75 -1.7) (layer F.SilkS) (width 0.12))
  (fp_line (start 0.75 -1.7) (end 6.75 -1.7) (layer F.SilkS) (width 0.12))
  (fp_line (start 6.75 -1.7) (end 6.75 -2.45) (layer F.SilkS) (width 0.12))
  (fp_line (start 6.75 -2.45) (end 0.75 -2.45) (layer F.SilkS) (width 0.12))
  (fp_line (start -2.55 -2.45) (end -2.55 -1.7) (layer F.SilkS) (width 0.12))
  (fp_line (start -2.55 -1.7) (end -0.75 -1.7) (layer F.SilkS) (width 0.12))
  (fp_line (start -0.75 -1.7) (end -0.75 -2.45) (layer F.SilkS) (width 0.12))
  (fp_line (start -0.75 -2.45) (end -2.55 -2.45) (layer F.SilkS) (width 0.12))
  (fp_line (start 8.25 -2.45) (end 8.25 -1.7) (layer F.SilkS) (width 0.12))
  (fp_line (start 8.25 -1.7) (end 10.05 -1.7) (layer F.SilkS) (width 0.12))
  (fp_line (start 10.05 -1.7) (end 10.05 -2.45) (layer F.SilkS) (width 0.12))
  (fp_line (start 10.05 -2.45) (end 8.25 -2.45) (layer F.SilkS) (width 0.12))
  (fp_line (start -2.55 -0.2) (end -1.8 -0.2) (layer F.SilkS) (width 0.12))
  (fp_line (start -1.8 -0.2) (end -1.8 2.75) (layer F.SilkS) (width 0.12))
  (fp_line (start -1.8 2.75) (end 3.75 2.75) (layer F.SilkS) (width 0.12))
  (fp_line (start 10.05 -0.2) (end 9.3 -0.2) (layer F.SilkS) (width 0.12))
  (fp_line (start 9.3 -0.2) (end 9.3 2.75) (layer F.SilkS) (width 0.12))
  (fp_line (start 9.3 2.75) (end 3.75 2.75) (layer F.SilkS) (width 0.12))
  (fp_line (start -1.6 -2.75) (end -2.85 -2.75) (layer F.SilkS) (width 0.12))
  (fp_line (start -2.85 -2.75) (end -2.85 -1.5) (layer F.SilkS) (width 0.12))
  (pad 4 thru_hole oval (at 7.5 0 270) (size 1.7 1.95) (drill 0.95) (layers *.Cu *.Mask) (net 48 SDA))
  (pad 3 thru_hole oval (at 5 0 270) (size 1.7 1.95) (drill 0.95) (layers *.Cu *.Mask) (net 49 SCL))
  (pad 2 thru_hole oval (at 2.5 0 270) (size 1.7 1.95) (drill 0.95) (layers *.Cu *.Mask) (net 12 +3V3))
  (pad 1 thru_hole roundrect (at 0 0 270) (size 1.7 1.95) (drill 0.95) (layers *.Cu *.Mask) (roundrect_rratio 0.147059) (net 2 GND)))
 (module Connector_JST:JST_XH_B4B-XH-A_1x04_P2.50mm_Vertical (layer F.Cu) (at 151.56 109.76 270)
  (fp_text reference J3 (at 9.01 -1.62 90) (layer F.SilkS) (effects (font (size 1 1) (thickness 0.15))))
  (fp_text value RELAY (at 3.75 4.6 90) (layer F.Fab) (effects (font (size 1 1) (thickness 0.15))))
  (fp_line (start -2.85 -2.75) (end -2.85 -1.5) (layer F.SilkS) (width 0.12))
  (fp_line (start -1.6 -2.75) (end -2.85 -2.75) (layer F.SilkS) (width 0.12))
  (fp_line (start 9.3 2.75) (end 3.75 2.75) (layer F.SilkS) (width 0.12))
  (fp_line (start 9.3 -0.2) (end 9.3 2.75) (layer F.SilkS) (width 0.12))
  (fp_line (start 10.05 -0.2) (end 9.3 -0.2) (layer F.SilkS) (width 0.12))
  (fp_line (start -1.8 2.75) (end 3.75 2.75) (layer F.SilkS) (width 0.12))
  (fp_line (start -1.8 -0.2) (end -1.8 2.75) (layer F.SilkS) (width 0.12))
  (fp_line (start -2.55 -0.2) (end -1.8 -0.2) (layer F.SilkS) (width 0.12))
  (fp_line (start 10.05 -2.45) (end 8.25 -2.45) (layer F.SilkS) (width 0.12))
  (fp_line (start 10.05 -1.7) (end 10.05 -2.45) (layer F.SilkS) (width 0.12))
  (fp_line (start 8.25 -1.7) (end 10.05 -1.7) (layer F.SilkS) (width 0.12))
  (fp_line (start 8.25 -2.45) (end 8.25 -1.7) (layer F.SilkS) (width 0.12))
  (fp_line (start -0.75 -2.45) (end -2.55 -2.45) (layer F.SilkS) (width 0.12))
  (fp_line (start -0.75 -1.7) (end -0.75 -2.45) (layer F.SilkS) (width 0.12))
  (fp_line (start -2.55 -1.7) (end -0.75 -1.7) (layer F.SilkS) (width 0.12))
  (fp_line (start -2.55 -2.45) (end -2.55 -1.7) (layer F.SilkS) (width 0.12))
  (fp_line (start 6.75 -2.45) (end 0.75 -2.45) (layer F.SilkS) (width 0.12))
  (fp_line (start 6.75 -1.7) (end 6.75 -2.45) (layer F.SilkS) (width 0.12))
  (fp_line (start 0.75 -1.7) (end 6.75 -1.7) (layer F.SilkS) (width 0.12))
  (fp_line (start 0.75 -2.45) (end 0.75 -1.7) (layer F.SilkS) (width 0.12))
  (fp_line (start 10.06 -2.46) (end -2.56 -2.46) (layer F.SilkS) (width 0.12))
  (fp_line (start 10.06 3.51) (end 10.06 -2.46) (layer F.SilkS) (width 0.12))
  (fp_line (start -2.56 3.51) (end 10.06 3.51) (layer F.SilkS) (width 0.12))
  (fp_line (start -2.56 -2.46) (end -2.56 3.51) (layer F.SilkS) (width 0.12))
  (pad 1 thru_hole roundrect (at 0 0 270) (size 1.7 1.95) (drill 0.95) (layers *.Cu *.Mask) (roundrect_rratio 0.147059) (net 2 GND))
  (pad 2 thru_hole oval (at 2.5 0 270) (size 1.7 1.95) (drill 0.95) (layers *.Cu *.Mask) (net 45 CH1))
  (pad 3 thru_hole oval (at 5 0 270) (size 1.7 1.95) (drill 0.95) (layers *.Cu *.Mask) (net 46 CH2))
  (pad 4 thru_hole oval (at 7.5 0 270) (size 1.7 1.95) (drill 0.95) (layers *.Cu *.Mask) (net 16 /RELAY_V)))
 (gr_line (start 155 87) (end 155 125.35) (layer Edge.Cuts) (width 0.1))
 (gr_line (start 127.72 87) (end 155 87) (layer Edge.Cuts) (width 0.1))
 (gr_line (start 127.72 125.35) (end 127.72 87) (layer Edge.Cuts) (width 0.1))
 (gr_line (start 155 125.35) (end 127.72 125.35) (layer Edge.Cuts) (width 0.1))
 (segment (start 143.305 118.99) (end 143.605 119.29) (width 0.2) (layer B.Cu) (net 18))
 (segment (start 143.305 117.6525) (end 143.305 118.99) (width 0.2) (layer B.Cu) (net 18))
 (segment (start 143.33 117.6275) (end 143.305 117.6525) (width 0.2) (layer B.Cu) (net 18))
 (via (at 143.605 119.29) (size 0.8) (drill 0.4) (layers F.Cu B.Cu) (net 18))
 (segment (start 143.3 121.216397) (end 143.3 121.23) (width 0.2) (layer F.Cu) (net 18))
 (segment (start 143.424999 121.091398) (end 143.3 121.216397) (width 0.2) (layer F.Cu) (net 18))
 (segment (start 143.424999 120.299999) (end 143.424999 121.091398) (width 0.2) (layer F.Cu) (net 18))
 (segment (start 143.605 120.119998) (end 143.424999 120.299999) (width 0.2) (layer F.Cu) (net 18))
 (segment (start 143.605 119.29) (end 143.605 120.119998) (width 0.2) (layer F.Cu) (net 18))
 (segment (start 142.855 118.99) (end 142.555 119.29) (width 0.2) (layer B.Cu) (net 17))
 (segment (start 142.83 117.6275) (end 142.855 117.6525) (width 0.2) (layer B.Cu) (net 17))
 (segment (start 142.855 117.6525) (end 142.855 118.99) (width 0.2) (layer B.Cu) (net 17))
 (via (at 142.555 119.29) (size 0.8) (drill 0.4) (layers F.Cu B.Cu) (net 17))
 (segment (start 142.774999 120.299999) (end 142.774999 121.105001) (width 0.2) (layer F.Cu) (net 17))
 (segment (start 143.155 119.919998) (end 142.774999 120.299999) (width 0.2) (layer F.Cu) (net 17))
 (segment (start 143.155 119.89) (end 143.155 119.919998) (width 0.2) (layer F.Cu) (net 17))
 (segment (start 142.555 119.29) (end 143.155 119.89) (width 0.2) (layer F.Cu) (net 17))
 (segment (start 142.774999 121.105001) (end 142.65 121.23) (width 0.2) (layer F.Cu) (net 17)))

